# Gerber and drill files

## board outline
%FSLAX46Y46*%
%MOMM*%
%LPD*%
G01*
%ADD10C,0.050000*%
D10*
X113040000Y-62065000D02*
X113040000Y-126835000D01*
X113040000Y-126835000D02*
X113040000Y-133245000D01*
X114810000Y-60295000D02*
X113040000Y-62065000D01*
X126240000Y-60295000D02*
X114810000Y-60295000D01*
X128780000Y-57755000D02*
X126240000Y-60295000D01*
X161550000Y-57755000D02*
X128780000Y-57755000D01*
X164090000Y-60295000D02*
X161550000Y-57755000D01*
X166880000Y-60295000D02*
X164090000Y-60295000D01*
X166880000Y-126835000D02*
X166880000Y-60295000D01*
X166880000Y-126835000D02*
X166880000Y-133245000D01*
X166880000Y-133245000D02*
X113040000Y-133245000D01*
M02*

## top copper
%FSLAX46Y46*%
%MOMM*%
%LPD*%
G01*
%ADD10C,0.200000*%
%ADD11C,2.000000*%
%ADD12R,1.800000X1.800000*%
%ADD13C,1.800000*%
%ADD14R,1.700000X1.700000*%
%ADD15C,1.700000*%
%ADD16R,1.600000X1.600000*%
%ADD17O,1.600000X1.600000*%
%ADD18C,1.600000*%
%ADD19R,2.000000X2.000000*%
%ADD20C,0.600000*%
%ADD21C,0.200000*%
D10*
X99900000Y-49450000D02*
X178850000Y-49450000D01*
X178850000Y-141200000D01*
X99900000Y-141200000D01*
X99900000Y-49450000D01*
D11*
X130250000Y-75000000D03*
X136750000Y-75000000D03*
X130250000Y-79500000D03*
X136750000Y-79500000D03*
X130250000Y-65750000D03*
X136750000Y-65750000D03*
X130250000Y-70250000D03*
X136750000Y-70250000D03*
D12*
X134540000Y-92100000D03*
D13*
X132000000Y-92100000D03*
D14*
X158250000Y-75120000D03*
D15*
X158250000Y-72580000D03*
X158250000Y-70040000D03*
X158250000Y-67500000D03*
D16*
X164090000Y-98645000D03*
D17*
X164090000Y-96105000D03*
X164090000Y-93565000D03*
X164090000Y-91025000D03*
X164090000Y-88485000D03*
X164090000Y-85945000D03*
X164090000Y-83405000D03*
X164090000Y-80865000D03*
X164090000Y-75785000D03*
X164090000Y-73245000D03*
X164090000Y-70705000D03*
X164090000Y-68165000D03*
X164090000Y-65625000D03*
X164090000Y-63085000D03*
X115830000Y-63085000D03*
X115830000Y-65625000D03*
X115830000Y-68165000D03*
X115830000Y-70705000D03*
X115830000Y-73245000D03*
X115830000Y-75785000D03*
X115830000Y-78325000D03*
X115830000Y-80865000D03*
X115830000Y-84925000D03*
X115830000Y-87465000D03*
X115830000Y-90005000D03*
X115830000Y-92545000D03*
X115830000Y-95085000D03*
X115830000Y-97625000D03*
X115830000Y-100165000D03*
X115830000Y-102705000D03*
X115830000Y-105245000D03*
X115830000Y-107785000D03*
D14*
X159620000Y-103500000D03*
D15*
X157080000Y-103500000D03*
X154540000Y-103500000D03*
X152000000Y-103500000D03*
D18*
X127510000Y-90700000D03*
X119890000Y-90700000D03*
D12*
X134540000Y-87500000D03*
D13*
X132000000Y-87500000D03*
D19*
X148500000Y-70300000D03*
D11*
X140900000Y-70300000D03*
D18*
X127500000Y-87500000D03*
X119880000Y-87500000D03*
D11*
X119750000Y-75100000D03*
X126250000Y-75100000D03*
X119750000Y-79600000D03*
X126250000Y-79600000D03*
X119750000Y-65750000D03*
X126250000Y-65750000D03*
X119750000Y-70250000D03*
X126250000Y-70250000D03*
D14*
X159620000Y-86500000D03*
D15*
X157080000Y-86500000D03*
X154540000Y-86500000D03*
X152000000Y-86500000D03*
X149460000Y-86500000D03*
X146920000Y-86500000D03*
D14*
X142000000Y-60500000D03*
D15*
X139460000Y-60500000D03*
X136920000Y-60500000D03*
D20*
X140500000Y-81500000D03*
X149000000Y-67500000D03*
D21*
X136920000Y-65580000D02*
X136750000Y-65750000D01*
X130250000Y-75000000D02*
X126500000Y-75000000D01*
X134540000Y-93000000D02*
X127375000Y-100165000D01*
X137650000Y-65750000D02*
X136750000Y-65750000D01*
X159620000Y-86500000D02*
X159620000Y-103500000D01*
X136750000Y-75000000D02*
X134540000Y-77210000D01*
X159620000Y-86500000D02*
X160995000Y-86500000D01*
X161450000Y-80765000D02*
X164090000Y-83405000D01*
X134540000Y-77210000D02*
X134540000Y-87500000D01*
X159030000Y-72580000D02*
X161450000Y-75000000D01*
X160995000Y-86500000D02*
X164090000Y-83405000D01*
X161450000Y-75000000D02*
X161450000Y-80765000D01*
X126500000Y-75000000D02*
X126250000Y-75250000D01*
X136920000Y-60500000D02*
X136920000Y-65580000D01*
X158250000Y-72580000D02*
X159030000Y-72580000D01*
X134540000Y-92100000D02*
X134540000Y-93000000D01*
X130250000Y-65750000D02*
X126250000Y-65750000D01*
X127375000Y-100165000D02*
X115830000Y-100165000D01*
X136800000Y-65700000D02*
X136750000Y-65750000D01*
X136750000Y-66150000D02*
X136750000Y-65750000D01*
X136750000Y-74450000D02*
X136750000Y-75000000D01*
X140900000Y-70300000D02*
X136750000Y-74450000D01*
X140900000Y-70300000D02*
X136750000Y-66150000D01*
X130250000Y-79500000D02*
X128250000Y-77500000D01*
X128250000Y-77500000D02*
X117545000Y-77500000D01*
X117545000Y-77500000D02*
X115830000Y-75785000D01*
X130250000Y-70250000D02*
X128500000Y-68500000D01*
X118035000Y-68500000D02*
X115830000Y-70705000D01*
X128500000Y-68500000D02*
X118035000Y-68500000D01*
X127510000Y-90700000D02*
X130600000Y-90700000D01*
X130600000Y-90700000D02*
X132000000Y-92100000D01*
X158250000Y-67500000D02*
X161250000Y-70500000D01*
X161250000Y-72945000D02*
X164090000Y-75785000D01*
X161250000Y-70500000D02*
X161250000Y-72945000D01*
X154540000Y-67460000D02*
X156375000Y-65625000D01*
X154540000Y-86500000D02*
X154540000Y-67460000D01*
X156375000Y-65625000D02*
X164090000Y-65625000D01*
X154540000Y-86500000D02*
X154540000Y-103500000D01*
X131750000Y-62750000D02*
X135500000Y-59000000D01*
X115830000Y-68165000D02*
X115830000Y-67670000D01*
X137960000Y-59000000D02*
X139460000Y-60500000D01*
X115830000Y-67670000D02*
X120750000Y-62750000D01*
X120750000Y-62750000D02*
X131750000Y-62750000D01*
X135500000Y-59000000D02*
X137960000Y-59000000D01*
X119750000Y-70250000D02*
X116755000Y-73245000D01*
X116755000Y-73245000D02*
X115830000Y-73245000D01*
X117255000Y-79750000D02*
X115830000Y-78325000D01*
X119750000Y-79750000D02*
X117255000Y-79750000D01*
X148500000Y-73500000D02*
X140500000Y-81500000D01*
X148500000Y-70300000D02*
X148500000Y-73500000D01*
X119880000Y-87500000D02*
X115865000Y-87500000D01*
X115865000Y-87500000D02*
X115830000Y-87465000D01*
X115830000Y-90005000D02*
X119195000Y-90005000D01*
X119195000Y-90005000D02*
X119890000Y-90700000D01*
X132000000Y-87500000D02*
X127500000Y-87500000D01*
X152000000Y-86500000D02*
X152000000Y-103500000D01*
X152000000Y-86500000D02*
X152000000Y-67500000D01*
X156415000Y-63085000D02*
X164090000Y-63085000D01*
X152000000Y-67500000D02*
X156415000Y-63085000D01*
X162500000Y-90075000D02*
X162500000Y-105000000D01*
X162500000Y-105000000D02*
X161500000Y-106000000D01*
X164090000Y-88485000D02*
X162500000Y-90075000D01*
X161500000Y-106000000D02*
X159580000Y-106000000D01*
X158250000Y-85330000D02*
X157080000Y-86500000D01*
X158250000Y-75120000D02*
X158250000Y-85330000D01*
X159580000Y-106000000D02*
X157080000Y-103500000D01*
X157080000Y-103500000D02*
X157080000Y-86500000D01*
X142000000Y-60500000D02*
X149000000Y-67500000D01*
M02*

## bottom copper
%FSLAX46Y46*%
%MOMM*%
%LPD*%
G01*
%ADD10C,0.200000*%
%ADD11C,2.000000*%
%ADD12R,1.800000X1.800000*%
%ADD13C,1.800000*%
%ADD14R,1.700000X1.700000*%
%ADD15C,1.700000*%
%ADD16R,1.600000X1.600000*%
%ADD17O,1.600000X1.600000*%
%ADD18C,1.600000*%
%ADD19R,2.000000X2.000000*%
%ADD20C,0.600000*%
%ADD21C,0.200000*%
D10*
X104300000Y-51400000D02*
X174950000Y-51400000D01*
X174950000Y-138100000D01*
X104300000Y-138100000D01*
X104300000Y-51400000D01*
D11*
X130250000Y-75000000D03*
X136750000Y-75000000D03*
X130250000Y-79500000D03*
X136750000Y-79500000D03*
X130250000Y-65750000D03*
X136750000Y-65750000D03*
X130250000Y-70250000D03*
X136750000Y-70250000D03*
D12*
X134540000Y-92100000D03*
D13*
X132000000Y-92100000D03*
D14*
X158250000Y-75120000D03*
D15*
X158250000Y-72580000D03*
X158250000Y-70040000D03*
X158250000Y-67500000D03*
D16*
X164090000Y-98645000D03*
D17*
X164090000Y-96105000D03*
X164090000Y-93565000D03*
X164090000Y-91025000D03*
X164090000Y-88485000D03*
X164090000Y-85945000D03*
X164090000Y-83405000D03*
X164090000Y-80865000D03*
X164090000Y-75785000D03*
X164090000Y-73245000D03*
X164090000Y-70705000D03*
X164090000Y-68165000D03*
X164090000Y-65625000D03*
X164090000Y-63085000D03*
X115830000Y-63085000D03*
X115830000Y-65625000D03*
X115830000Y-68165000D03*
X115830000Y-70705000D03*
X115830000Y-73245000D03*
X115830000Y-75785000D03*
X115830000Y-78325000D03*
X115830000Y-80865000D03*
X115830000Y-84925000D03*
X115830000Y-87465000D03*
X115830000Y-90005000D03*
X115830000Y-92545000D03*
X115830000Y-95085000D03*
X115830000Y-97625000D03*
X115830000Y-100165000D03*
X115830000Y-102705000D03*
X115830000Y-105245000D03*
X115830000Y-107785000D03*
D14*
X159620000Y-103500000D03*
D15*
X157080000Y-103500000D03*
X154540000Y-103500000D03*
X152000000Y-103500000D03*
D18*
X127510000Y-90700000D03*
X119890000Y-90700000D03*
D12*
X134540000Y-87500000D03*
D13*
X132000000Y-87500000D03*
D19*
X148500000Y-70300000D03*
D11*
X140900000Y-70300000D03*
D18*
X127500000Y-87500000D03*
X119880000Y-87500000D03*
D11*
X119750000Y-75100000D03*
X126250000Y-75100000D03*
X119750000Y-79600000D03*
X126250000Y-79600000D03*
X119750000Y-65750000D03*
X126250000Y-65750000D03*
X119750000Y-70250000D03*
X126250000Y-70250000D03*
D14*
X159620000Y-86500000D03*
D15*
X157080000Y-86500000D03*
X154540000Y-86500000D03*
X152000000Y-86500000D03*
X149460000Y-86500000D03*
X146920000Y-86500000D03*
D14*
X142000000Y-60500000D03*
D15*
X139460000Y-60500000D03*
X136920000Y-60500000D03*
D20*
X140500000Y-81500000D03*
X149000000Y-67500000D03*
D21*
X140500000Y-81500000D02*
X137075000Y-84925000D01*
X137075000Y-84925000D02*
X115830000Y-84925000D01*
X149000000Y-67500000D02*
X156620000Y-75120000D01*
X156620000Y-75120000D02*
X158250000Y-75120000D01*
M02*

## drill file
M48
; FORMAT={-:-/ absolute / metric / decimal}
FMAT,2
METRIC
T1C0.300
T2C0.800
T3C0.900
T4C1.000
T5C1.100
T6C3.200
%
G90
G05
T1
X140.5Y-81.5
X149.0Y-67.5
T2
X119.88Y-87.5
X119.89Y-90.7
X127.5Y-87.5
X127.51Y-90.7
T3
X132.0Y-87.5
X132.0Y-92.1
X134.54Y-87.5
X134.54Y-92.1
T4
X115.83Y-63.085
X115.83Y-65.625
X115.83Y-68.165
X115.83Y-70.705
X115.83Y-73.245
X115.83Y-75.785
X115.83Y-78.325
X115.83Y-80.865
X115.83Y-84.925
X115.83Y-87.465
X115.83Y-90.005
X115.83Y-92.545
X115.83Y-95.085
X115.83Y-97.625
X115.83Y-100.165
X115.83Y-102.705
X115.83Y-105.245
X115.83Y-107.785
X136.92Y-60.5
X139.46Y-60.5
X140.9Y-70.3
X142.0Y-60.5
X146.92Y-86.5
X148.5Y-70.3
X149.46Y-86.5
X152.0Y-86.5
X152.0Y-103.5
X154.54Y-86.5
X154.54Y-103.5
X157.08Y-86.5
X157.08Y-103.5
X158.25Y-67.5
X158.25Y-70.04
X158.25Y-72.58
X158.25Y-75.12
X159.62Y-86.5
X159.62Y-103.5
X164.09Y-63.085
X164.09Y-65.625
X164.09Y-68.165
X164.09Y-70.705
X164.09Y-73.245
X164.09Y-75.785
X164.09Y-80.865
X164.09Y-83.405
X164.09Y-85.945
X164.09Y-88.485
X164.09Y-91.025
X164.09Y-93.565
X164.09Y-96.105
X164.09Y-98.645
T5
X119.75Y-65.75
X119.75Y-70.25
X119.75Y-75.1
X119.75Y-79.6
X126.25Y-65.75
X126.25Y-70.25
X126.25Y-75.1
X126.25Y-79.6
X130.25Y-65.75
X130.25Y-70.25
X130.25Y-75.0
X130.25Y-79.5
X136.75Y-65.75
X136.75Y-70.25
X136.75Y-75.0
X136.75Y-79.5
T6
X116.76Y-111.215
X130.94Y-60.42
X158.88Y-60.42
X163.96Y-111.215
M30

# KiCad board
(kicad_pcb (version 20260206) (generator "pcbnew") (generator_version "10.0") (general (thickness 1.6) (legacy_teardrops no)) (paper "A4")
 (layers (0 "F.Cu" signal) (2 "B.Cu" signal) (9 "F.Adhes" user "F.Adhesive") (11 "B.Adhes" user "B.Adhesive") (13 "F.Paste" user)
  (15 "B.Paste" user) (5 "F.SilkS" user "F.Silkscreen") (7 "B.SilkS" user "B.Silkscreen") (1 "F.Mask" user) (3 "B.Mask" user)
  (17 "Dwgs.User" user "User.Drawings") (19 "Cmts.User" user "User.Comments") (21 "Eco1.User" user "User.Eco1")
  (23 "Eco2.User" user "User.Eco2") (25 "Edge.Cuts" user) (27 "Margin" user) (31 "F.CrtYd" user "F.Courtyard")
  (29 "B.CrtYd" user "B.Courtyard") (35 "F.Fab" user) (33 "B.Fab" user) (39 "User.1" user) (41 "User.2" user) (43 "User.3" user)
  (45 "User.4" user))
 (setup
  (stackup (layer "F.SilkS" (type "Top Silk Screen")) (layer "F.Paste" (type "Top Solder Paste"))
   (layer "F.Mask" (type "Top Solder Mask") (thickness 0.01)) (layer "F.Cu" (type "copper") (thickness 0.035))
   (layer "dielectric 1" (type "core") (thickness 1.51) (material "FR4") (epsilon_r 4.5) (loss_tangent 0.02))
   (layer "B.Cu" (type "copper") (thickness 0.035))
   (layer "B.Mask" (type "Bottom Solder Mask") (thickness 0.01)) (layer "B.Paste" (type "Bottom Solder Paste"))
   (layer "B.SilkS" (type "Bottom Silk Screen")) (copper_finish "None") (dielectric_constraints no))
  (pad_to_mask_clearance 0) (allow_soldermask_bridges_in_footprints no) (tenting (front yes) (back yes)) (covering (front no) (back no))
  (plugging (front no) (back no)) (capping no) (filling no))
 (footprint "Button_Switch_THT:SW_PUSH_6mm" (layer "F.Cu") (at 130.25 75)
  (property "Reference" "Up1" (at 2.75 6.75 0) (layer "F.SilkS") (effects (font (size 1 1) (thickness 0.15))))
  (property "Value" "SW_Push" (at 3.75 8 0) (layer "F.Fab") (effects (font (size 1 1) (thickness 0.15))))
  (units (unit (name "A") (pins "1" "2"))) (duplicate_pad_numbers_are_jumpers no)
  (pad "1" thru_hole circle (at 0 0 90) (size 2 2) (drill 1.1) (layers "*.Cu" "*.Mask") (remove_unused_layers no) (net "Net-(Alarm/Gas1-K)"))
  (pad "1" thru_hole circle (at 6.5 0 90) (size 2 2) (drill 1.1) (layers "*.Cu" "*.Mask") (remove_unused_layers no)
   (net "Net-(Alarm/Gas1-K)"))
  (pad "2" thru_hole circle (at 0 4.5 90) (size 2 2) (drill 1.1) (layers "*.Cu" "*.Mask") (remove_unused_layers no) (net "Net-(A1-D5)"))
  (pad "2" thru_hole circle (at 6.5 4.5 90) (size 2 2) (drill 1.1) (layers "*.Cu" "*.Mask") (remove_unused_layers no) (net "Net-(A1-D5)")))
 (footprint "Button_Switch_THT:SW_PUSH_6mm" (layer "F.Cu") (at 130.25 65.75)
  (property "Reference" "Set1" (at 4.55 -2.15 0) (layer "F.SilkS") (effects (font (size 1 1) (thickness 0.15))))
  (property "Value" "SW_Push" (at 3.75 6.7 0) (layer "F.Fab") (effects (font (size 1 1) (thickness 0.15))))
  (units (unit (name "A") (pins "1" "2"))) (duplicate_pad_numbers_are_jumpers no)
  (pad "1" thru_hole circle (at 0 0 90) (size 2 2) (drill 1.1) (layers "*.Cu" "*.Mask") (remove_unused_layers no) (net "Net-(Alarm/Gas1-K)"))
  (pad "1" thru_hole circle (at 6.5 0 90) (size 2 2) (drill 1.1) (layers "*.Cu" "*.Mask") (remove_unused_layers no)
   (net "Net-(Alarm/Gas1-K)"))
  (pad "2" thru_hole circle (at 0 4.5 90) (size 2 2) (drill 1.1) (layers "*.Cu" "*.Mask") (remove_unused_layers no) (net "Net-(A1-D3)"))
  (pad "2" thru_hole circle (at 6.5 4.5 90) (size 2 2) (drill 1.1) (layers "*.Cu" "*.Mask") (remove_unused_layers no) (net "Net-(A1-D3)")))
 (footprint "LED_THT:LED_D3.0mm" (layer "F.Cu") (at 134.54 92.1 180)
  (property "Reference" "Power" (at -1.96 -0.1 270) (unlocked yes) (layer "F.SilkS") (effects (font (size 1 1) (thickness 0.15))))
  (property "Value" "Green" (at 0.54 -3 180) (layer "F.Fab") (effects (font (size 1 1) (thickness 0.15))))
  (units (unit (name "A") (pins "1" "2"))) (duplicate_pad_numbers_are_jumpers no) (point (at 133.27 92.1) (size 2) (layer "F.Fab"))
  (pad "1" thru_hole rect (at 0 0 180) (size 1.8 1.8) (drill 0.9) (layers "*.Cu" "*.Mask") (remove_unused_layers no)
   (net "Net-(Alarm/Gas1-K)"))
  (pad "2" thru_hole circle (at 2.54 0 180) (size 1.8 1.8) (drill 0.9) (layers "*.Cu" "*.Mask") (remove_unused_layers no)
   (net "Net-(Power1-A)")))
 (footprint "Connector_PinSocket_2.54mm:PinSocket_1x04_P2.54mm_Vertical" (layer "F.Cu") (at 158.25 75.12 180)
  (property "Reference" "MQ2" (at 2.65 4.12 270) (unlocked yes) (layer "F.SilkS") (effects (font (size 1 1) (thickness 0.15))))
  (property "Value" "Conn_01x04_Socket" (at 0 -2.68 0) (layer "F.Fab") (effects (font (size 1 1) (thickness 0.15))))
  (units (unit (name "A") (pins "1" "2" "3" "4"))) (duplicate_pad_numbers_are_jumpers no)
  (pad "1" thru_hole rect (at 0 0 180) (size 1.7 1.7) (drill 1) (layers "*.Cu" "*.Mask") (remove_unused_layers no) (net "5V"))
  (pad "2" thru_hole circle (at 0 2.54 180) (size 1.7 1.7) (drill 1) (layers "*.Cu" "*.Mask") (remove_unused_layers no)
   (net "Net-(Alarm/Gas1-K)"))
  (pad "3" thru_hole circle (at 0 5.08 180) (size 1.7 1.7) (drill 1) (layers "*.Cu" "*.Mask") (remove_unused_layers no)
   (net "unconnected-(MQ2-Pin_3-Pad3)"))
  (pad "4" thru_hole circle (at 0 7.62 180) (size 1.7 1.7) (drill 1) (layers "*.Cu" "*.Mask") (remove_unused_layers no) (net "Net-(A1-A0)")))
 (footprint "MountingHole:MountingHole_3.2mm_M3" (layer "F.Cu") (at 163.96 111.215)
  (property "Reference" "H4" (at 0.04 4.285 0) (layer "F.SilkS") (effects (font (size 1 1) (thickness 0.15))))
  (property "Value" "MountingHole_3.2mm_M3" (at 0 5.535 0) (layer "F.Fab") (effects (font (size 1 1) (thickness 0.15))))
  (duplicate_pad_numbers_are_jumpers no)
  (pad "" np_thru_hole circle (at 0 0) (size 3.2 3.2) (drill 3.2) (layers "*.Cu" "*.Mask")))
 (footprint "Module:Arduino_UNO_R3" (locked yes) (layer "F.Cu") (at 116.09 98.645 90)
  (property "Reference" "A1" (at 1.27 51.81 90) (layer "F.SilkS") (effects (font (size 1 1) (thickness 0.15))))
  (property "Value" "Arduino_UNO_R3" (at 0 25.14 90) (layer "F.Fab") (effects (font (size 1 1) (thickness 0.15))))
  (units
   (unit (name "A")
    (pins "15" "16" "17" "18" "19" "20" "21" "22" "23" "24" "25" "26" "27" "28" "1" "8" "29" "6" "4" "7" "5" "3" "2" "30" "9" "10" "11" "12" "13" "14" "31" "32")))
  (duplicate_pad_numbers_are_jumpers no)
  (fp_line (start 36.58 -3.05) (end -28.19 -3.05) (stroke (width 0.05) (type solid)) (layer "Edge.Cuts"))
  (fp_line (start -28.19 -3.05) (end -34.6 -3.05) (stroke (width 0.05) (type default)) (layer "Edge.Cuts"))
  (fp_line (start 38.35 -1.28) (end 36.58 -3.05) (stroke (width 0.05) (type solid)) (layer "Edge.Cuts"))
  (fp_line (start 38.35 10.15) (end 38.35 -1.28) (stroke (width 0.05) (type solid)) (layer "Edge.Cuts"))
  (fp_line (start 40.89 12.69) (end 38.35 10.15) (stroke (width 0.05) (type solid)) (layer "Edge.Cuts"))
  (fp_line (start 40.89 45.46) (end 40.89 12.69) (stroke (width 0.05) (type solid)) (layer "Edge.Cuts"))
  (fp_line (start 38.35 48) (end 40.89 45.46) (stroke (width 0.05) (type solid)) (layer "Edge.Cuts"))
  (fp_line (start 38.35 50.79) (end 38.35 48) (stroke (width 0.05) (type solid)) (layer "Edge.Cuts"))
  (fp_line (start -28.19 50.79) (end 38.35 50.79) (stroke (width 0.05) (type solid)) (layer "Edge.Cuts"))
  (fp_line (start -28.19 50.79) (end -34.6 50.79) (stroke (width 0.05) (type default)) (layer "Edge.Cuts"))
  (fp_line (start -34.6 50.79) (end -34.6 -3.05) (stroke (width 0.05) (type default)) (layer "Edge.Cuts"))
  (pad "1" thru_hole rect (at 0 48) (size 1.6 1.6) (drill 1) (layers "*.Cu" "*.Mask") (remove_unused_layers no)
   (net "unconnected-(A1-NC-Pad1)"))
  (pad "2" thru_hole oval (at 2.54 48) (size 1.6 1.6) (drill 1) (layers "*.Cu" "*.Mask") (remove_unused_layers no)
   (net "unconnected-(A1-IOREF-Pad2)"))
  (pad "3" thru_hole oval (at 5.08 48) (size 1.6 1.6) (drill 1) (layers "*.Cu" "*.Mask") (remove_unused_layers no)
   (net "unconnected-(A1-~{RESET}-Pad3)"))
  (pad "4" thru_hole oval (at 7.62 48) (size 1.6 1.6) (drill 1) (layers "*.Cu" "*.Mask") (remove_unused_layers no)
   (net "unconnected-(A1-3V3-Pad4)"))
  (pad "5" thru_hole oval (at 10.16 48) (size 1.6 1.6) (drill 1) (layers "*.Cu" "*.Mask") (remove_unused_layers no) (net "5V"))
  (pad "6" thru_hole oval (at 12.7 48) (size 1.6 1.6) (drill 1) (layers "*.Cu" "*.Mask") (remove_unused_layers no) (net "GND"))
  (pad "7" thru_hole oval (at 15.24 48) (size 1.6 1.6) (drill 1) (layers "*.Cu" "*.Mask") (remove_unused_layers no)
   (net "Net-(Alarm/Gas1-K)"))
  (pad "8" thru_hole oval (at 17.78 48) (size 1.6 1.6) (drill 1) (layers "*.Cu" "*.Mask") (remove_unused_layers no)
   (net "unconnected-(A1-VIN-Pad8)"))
  (pad "9" thru_hole oval (at 22.86 48) (size 1.6 1.6) (drill 1) (layers "*.Cu" "*.Mask") (remove_unused_layers no) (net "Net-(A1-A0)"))
  (pad "10" thru_hole oval (at 25.4 48) (size 1.6 1.6) (drill 1) (layers "*.Cu" "*.Mask") (remove_unused_layers no)
   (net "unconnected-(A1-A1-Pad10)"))
  (pad "11" thru_hole oval (at 27.94 48) (size 1.6 1.6) (drill 1) (layers "*.Cu" "*.Mask") (remove_unused_layers no)
   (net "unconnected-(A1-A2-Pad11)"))
  (pad "12" thru_hole oval (at 30.48 48) (size 1.6 1.6) (drill 1) (layers "*.Cu" "*.Mask") (remove_unused_layers no)
   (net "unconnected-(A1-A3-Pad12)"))
  (pad "13" thru_hole oval (at 33.02 48) (size 1.6 1.6) (drill 1) (layers "*.Cu" "*.Mask") (remove_unused_layers no)
   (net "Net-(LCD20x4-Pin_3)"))
  (pad "14" thru_hole oval (at 35.56 48) (size 1.6 1.6) (drill 1) (layers "*.Cu" "*.Mask") (remove_unused_layers no)
   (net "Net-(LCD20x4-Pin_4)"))
  (pad "15" thru_hole oval (at 35.56 -0.26) (size 1.6 1.6) (drill 1) (layers "*.Cu" "*.Mask") (remove_unused_layers no)
   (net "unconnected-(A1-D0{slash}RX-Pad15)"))
  (pad "16" thru_hole oval (at 33.02 -0.26) (size 1.6 1.6) (drill 1) (layers "*.Cu" "*.Mask") (remove_unused_layers no)
   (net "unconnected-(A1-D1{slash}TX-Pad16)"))
  (pad "17" thru_hole oval (at 30.48 -0.26) (size 1.6 1.6) (drill 1) (layers "*.Cu" "*.Mask") (remove_unused_layers no) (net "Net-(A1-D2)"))
  (pad "18" thru_hole oval (at 27.94 -0.26) (size 1.6 1.6) (drill 1) (layers "*.Cu" "*.Mask") (remove_unused_layers no) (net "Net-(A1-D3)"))
  (pad "19" thru_hole oval (at 25.4 -0.26) (size 1.6 1.6) (drill 1) (layers "*.Cu" "*.Mask") (remove_unused_layers no) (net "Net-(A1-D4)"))
  (pad "20" thru_hole oval (at 22.86 -0.26) (size 1.6 1.6) (drill 1) (layers "*.Cu" "*.Mask") (remove_unused_layers no) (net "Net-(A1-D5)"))
  (pad "21" thru_hole oval (at 20.32 -0.26) (size 1.6 1.6) (drill 1) (layers "*.Cu" "*.Mask") (remove_unused_layers no) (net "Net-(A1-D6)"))
  (pad "22" thru_hole oval (at 17.78 -0.26) (size 1.6 1.6) (drill 1) (layers "*.Cu" "*.Mask") (remove_unused_layers no)
   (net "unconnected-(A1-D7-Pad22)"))
  (pad "23" thru_hole oval (at 13.72 -0.26) (size 1.6 1.6) (drill 1) (layers "*.Cu" "*.Mask") (remove_unused_layers no) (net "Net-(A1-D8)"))
  (pad "24" thru_hole oval (at 11.18 -0.26) (size 1.6 1.6) (drill 1) (layers "*.Cu" "*.Mask") (remove_unused_layers no) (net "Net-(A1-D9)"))
  (pad "25" thru_hole oval (at 8.64 -0.26) (size 1.6 1.6) (drill 1) (layers "*.Cu" "*.Mask") (remove_unused_layers no) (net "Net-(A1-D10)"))
  (pad "26" thru_hole oval (at 6.1 -0.26) (size 1.6 1.6) (drill 1) (layers "*.Cu" "*.Mask") (remove_unused_layers no)
   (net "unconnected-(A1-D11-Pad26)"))
  (pad "27" thru_hole oval (at 3.56 -0.26) (size 1.6 1.6) (drill 1) (layers "*.Cu" "*.Mask") (remove_unused_layers no)
   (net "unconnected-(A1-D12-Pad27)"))
  (pad "28" thru_hole oval (at 1.02 -0.26) (size 1.6 1.6) (drill 1) (layers "*.Cu" "*.Mask") (remove_unused_layers no)
   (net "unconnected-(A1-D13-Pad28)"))
  (pad "29" thru_hole oval (at -1.52 -0.26) (size 1.6 1.6) (drill 1) (layers "*.Cu" "*.Mask") (remove_unused_layers no)
   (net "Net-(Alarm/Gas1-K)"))
  (pad "30" thru_hole oval (at -4.06 -0.26) (size 1.6 1.6) (drill 1) (layers "*.Cu" "*.Mask") (remove_unused_layers no)
   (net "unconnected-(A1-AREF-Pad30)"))
  (pad "31" thru_hole oval (at -6.6 -0.26) (size 1.6 1.6) (drill 1) (layers "*.Cu" "*.Mask") (remove_unused_layers no)
   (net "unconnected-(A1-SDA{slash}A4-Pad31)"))
  (pad "32" thru_hole oval (at -9.14 -0.26) (size 1.6 1.6) (drill 1) (layers "*.Cu" "*.Mask") (remove_unused_layers no)
   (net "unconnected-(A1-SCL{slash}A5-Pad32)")))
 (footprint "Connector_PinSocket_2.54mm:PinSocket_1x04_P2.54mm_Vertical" (layer "F.Cu") (at 159.62 103.5 -90)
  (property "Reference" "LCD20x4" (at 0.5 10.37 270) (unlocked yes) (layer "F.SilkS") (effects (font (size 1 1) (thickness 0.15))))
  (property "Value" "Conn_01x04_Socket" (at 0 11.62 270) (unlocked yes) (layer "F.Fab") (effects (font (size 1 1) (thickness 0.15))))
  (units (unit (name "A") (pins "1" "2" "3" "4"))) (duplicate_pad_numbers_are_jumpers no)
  (pad "1" thru_hole rect (at 0 0 270) (size 1.7 1.7) (drill 1) (layers "*.Cu" "*.Mask") (remove_unused_layers no)
   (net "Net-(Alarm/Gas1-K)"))
  (pad "2" thru_hole circle (at 0 2.54 270) (size 1.7 1.7) (drill 1) (layers "*.Cu" "*.Mask") (remove_unused_layers no) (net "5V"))
  (pad "3" thru_hole circle (at 0 5.08 270) (size 1.7 1.7) (drill 1) (layers "*.Cu" "*.Mask") (remove_unused_layers no)
   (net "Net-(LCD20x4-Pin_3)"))
  (pad "4" thru_hole circle (at 0 7.62 270) (size 1.7 1.7) (drill 1) (layers "*.Cu" "*.Mask") (remove_unused_layers no)
   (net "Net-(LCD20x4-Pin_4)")))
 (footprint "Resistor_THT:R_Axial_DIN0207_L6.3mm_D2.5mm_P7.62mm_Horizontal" (layer "F.Cu") (at 127.51 90.7 180)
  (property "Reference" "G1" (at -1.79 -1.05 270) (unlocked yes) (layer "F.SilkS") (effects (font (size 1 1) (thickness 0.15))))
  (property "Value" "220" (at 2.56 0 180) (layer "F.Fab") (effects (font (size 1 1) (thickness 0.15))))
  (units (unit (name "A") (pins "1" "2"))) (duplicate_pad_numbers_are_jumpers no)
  (pad "1" thru_hole circle (at 0 0 180) (size 1.6 1.6) (drill 0.8) (layers "*.Cu" "*.Mask") (remove_unused_layers no)
   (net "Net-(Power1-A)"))
  (pad "2" thru_hole circle (at 7.62 0 180) (size 1.6 1.6) (drill 0.8) (layers "*.Cu" "*.Mask") (remove_unused_layers no)
   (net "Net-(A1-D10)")))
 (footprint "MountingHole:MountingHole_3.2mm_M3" (layer "F.Cu") (at 116.76 111.215)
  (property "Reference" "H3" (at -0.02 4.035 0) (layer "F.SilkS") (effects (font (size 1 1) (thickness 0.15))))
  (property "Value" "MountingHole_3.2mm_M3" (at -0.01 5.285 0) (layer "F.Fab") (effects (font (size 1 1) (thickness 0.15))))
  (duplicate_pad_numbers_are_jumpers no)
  (pad "" np_thru_hole circle (at 0 0) (size 3.2 3.2) (drill 3.2) (layers "*.Cu" "*.Mask")))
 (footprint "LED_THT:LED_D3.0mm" (layer "F.Cu") (at 134.54 87.5 180)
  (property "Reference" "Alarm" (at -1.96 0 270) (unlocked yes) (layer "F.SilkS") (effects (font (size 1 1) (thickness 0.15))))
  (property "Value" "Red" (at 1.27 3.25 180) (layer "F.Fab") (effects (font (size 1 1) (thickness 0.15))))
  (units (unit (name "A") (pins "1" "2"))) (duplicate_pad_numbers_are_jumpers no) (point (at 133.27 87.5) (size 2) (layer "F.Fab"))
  (pad "1" thru_hole rect (at 0 0 180) (size 1.8 1.8) (drill 0.9) (layers "*.Cu" "*.Mask") (remove_unused_layers no)
   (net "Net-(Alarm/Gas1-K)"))
  (pad "2" thru_hole circle (at 2.54 0 180) (size 1.8 1.8) (drill 0.9) (layers "*.Cu" "*.Mask") (remove_unused_layers no)
   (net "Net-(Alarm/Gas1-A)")))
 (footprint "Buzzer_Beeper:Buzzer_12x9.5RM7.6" (layer "F.Cu") (at 148.5 70.3 180)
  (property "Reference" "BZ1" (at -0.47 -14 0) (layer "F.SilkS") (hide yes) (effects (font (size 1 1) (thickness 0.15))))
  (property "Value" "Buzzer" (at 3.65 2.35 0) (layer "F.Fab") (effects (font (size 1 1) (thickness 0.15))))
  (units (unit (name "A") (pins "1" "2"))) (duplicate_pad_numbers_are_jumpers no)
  (pad "1" thru_hole rect (at 0 0 180) (size 2 2) (drill 1) (layers "*.Cu" "*.Mask") (remove_unused_layers no) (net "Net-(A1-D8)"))
  (pad "2" thru_hole circle (at 7.6 0 180) (size 2 2) (drill 1) (layers "*.Cu" "*.Mask") (remove_unused_layers no)
   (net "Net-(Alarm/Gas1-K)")))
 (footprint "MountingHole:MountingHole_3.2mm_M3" (layer "F.Cu") (at 158.88 60.42)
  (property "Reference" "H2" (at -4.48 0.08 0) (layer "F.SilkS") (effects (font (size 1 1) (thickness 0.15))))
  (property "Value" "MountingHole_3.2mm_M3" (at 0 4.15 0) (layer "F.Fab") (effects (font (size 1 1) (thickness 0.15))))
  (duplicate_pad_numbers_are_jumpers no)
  (pad "" np_thru_hole circle (at 0 0) (size 3.2 3.2) (drill 3.2) (layers "*.Cu" "*.Mask")))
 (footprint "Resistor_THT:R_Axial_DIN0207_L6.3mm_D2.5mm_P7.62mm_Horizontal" (layer "F.Cu") (at 127.5 87.5 180)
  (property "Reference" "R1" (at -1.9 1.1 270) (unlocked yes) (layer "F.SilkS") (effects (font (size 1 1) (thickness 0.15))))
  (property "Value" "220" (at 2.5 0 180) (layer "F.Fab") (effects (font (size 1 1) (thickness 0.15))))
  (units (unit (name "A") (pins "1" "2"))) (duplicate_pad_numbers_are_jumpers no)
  (pad "1" thru_hole circle (at 0 0 180) (size 1.6 1.6) (drill 0.8) (layers "*.Cu" "*.Mask") (remove_unused_layers no)
   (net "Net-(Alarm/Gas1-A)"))
  (pad "2" thru_hole circle (at 7.62 0 180) (size 1.6 1.6) (drill 0.8) (layers "*.Cu" "*.Mask") (remove_unused_layers no)
   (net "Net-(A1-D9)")))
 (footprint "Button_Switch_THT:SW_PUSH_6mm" (layer "F.Cu") (at 119.75 75.1)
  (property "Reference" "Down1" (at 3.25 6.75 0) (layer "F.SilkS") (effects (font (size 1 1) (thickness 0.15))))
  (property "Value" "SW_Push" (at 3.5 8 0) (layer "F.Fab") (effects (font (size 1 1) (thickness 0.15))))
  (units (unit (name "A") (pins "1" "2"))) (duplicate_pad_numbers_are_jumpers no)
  (pad "1" thru_hole circle (at 0 0 90) (size 2 2) (drill 1.1) (layers "*.Cu" "*.Mask") (remove_unused_layers no) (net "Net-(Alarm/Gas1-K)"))
  (pad "1" thru_hole circle (at 6.5 0 90) (size 2 2) (drill 1.1) (layers "*.Cu" "*.Mask") (remove_unused_layers no)
   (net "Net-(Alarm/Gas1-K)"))
  (pad "2" thru_hole circle (at 0 4.5 90) (size 2 2) (drill 1.1) (layers "*.Cu" "*.Mask") (remove_unused_layers no) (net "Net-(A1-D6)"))
  (pad "2" thru_hole circle (at 6.5 4.5 90) (size 2 2) (drill 1.1) (layers "*.Cu" "*.Mask") (remove_unused_layers no) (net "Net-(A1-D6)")))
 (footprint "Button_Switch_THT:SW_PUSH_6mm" (layer "F.Cu") (at 119.75 65.75)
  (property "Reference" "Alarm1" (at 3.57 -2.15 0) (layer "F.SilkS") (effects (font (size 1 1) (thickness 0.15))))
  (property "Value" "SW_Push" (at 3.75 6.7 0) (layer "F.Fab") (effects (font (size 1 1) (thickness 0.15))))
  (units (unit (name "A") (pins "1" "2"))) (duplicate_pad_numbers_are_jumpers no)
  (pad "1" thru_hole circle (at 0 0 90) (size 2 2) (drill 1.1) (layers "*.Cu" "*.Mask") (remove_unused_layers no) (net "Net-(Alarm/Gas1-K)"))
  (pad "1" thru_hole circle (at 6.5 0 90) (size 2 2) (drill 1.1) (layers "*.Cu" "*.Mask") (remove_unused_layers no)
   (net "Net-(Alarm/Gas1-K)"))
  (pad "2" thru_hole circle (at 0 4.5 90) (size 2 2) (drill 1.1) (layers "*.Cu" "*.Mask") (remove_unused_layers no) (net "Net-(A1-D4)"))
  (pad "2" thru_hole circle (at 6.5 4.5 90) (size 2 2) (drill 1.1) (layers "*.Cu" "*.Mask") (remove_unused_layers no) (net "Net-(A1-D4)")))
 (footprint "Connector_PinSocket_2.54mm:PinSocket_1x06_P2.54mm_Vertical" (layer "F.Cu") (at 159.62 86.5 -90)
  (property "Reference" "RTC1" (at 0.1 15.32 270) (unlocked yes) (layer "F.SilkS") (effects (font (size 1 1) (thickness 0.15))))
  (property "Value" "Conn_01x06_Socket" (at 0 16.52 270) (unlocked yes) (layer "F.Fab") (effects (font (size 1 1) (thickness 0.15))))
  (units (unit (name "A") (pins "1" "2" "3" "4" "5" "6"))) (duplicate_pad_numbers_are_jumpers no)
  (pad "1" thru_hole rect (at 0 0 270) (size 1.7 1.7) (drill 1) (layers "*.Cu" "*.Mask") (remove_unused_layers no)
   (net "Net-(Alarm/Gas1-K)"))
  (pad "2" thru_hole circle (at 0 2.54 270) (size 1.7 1.7) (drill 1) (layers "*.Cu" "*.Mask") (remove_unused_layers no) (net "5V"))
  (pad "3" thru_hole circle (at 0 5.08 270) (size 1.7 1.7) (drill 1) (layers "*.Cu" "*.Mask") (remove_unused_layers no)
   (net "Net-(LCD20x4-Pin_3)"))
  (pad "4" thru_hole circle (at 0 7.62 270) (size 1.7 1.7) (drill 1) (layers "*.Cu" "*.Mask") (remove_unused_layers no)
   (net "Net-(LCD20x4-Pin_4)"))
  (pad "5" thru_hole circle (at 0 10.16 270) (size 1.7 1.7) (drill 1) (layers "*.Cu" "*.Mask") (remove_unused_layers no)
   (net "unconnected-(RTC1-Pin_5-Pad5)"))
  (pad "6" thru_hole circle (at 0 12.7 270) (size 1.7 1.7) (drill 1) (layers "*.Cu" "*.Mask") (remove_unused_layers no)
   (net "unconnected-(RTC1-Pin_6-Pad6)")))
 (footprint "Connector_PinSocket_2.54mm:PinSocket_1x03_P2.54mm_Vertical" (layer "F.Cu") (at 142 60.5 -90)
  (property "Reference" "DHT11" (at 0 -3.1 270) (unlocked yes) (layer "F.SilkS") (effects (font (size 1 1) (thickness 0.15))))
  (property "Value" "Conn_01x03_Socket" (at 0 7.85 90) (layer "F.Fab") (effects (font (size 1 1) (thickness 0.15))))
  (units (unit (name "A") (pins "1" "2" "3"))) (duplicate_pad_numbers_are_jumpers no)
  (pad "1" thru_hole rect (at 0 0 270) (size 1.7 1.7) (drill 1) (layers "*.Cu" "*.Mask") (remove_unused_layers no) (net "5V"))
  (pad "2" thru_hole circle (at 0 2.54 270) (size 1.7 1.7) (drill 1) (layers "*.Cu" "*.Mask") (remove_unused_layers no) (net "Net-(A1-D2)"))
  (pad "3" thru_hole circle (at 0 5.08 270) (size 1.7 1.7) (drill 1) (layers "*.Cu" "*.Mask") (remove_unused_layers no)
   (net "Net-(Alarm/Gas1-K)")))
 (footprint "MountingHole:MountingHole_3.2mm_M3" (layer "F.Cu") (at 130.94 60.42)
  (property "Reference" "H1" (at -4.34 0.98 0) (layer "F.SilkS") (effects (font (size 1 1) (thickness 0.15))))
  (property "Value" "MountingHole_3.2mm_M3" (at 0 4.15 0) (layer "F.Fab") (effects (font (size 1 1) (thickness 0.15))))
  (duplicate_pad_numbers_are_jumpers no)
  (pad "" np_thru_hole circle (at 0 0) (size 3.2 3.2) (drill 3.2) (layers "*.Cu" "*.Mask")))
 (gr_rect (start 99.9 49.45) (end 178.85 141.2) (stroke (width 0.2) (type default)) (fill no) (layers "F.Cu" "F.Mask"))
 (gr_rect (start 104.3 51.4) (end 174.95 138.1) (stroke (width 0.2) (type default)) (fill no) (layer "B.Cu"))
 (segment (start 136.92 65.58) (end 136.75 65.75) (width 0.2) (layer "F.Cu") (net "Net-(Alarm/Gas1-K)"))
 (segment (start 130.25 75) (end 126.5 75) (width 0.2) (layer "F.Cu") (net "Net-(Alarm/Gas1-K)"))
 (segment (start 134.54 93) (end 127.375 100.165) (width 0.2) (layer "F.Cu") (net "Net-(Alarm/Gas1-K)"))
 (segment (start 137.65 65.75) (end 136.75 65.75) (width 0.2) (layer "F.Cu") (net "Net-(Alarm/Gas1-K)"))
 (segment (start 159.62 86.5) (end 159.62 103.5) (width 0.2) (layer "F.Cu") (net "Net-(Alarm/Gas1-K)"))
 (segment (start 136.75 75) (end 134.54 77.21) (width 0.2) (layer "F.Cu") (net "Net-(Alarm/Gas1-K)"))
 (segment (start 159.62 86.5) (end 160.995 86.5) (width 0.2) (layer "F.Cu") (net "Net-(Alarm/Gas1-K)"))
 (segment (start 161.45 80.765) (end 164.09 83.405) (width 0.2) (layer "F.Cu") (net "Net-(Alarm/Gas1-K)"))
 (segment (start 134.54 77.21) (end 134.54 87.5) (width 0.2) (layer "F.Cu") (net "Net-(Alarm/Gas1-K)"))
 (segment (start 159.03 72.58) (end 161.45 75) (width 0.2) (layer "F.Cu") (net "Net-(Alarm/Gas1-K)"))
 (segment (start 160.995 86.5) (end 164.09 83.405) (width 0.2) (layer "F.Cu") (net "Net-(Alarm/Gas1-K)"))
 (segment (start 161.45 75) (end 161.45 80.765) (width 0.2) (layer "F.Cu") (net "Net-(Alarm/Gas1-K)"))
 (segment (start 126.5 75) (end 126.25 75.25) (width 0.2) (layer "F.Cu") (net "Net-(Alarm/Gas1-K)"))
 (segment (start 136.92 60.5) (end 136.92 65.58) (width 0.2) (layer "F.Cu") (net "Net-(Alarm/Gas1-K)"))
 (segment (start 158.25 72.58) (end 159.03 72.58) (width 0.2) (layer "F.Cu") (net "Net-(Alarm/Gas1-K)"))
 (segment (start 134.54 92.1) (end 134.54 93) (width 0.2) (layer "F.Cu") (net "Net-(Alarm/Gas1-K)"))
 (segment (start 130.25 65.75) (end 126.25 65.75) (width 0.2) (layer "F.Cu") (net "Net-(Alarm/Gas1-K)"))
 (segment (start 127.375 100.165) (end 115.83 100.165) (width 0.2) (layer "F.Cu") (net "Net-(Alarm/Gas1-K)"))
 (segment (start 136.8 65.7) (end 136.75 65.75) (width 0.2) (layer "F.Cu") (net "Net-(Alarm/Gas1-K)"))
 (segment (start 136.75 66.15) (end 136.75 65.75) (width 0.2) (layer "F.Cu") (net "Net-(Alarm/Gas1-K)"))
 (segment (start 136.75 74.45) (end 136.75 75) (width 0.2) (layer "F.Cu") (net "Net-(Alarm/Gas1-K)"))
 (segment (start 140.9 70.3) (end 136.75 74.45) (width 0.2) (layer "F.Cu") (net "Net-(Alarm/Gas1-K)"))
 (segment (start 140.9 70.3) (end 136.75 66.15) (width 0.2) (layer "F.Cu") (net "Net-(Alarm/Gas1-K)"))
 (segment (start 130.25 79.5) (end 128.25 77.5) (width 0.2) (layer "F.Cu") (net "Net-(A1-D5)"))
 (segment (start 128.25 77.5) (end 117.545 77.5) (width 0.2) (layer "F.Cu") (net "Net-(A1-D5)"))
 (segment (start 117.545 77.5) (end 115.83 75.785) (width 0.2) (layer "F.Cu") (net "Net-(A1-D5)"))
 (segment (start 130.25 70.25) (end 128.5 68.5) (width 0.2) (layer "F.Cu") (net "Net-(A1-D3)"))
 (segment (start 118.035 68.5) (end 115.83 70.705) (width 0.2) (layer "F.Cu") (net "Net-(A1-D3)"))
 (segment (start 128.5 68.5) (end 118.035 68.5) (width 0.2) (layer "F.Cu") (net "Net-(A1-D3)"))
 (segment (start 127.51 90.7) (end 130.6 90.7) (width 0.2) (layer "F.Cu") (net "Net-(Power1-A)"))
 (segment (start 130.6 90.7) (end 132 92.1) (width 0.2) (layer "F.Cu") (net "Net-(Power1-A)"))
 (segment (start 158.25 67.5) (end 161.25 70.5) (width 0.2) (layer "F.Cu") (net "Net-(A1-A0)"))
 (segment (start 161.25 72.945) (end 164.09 75.785) (width 0.2) (layer "F.Cu") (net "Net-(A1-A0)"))
 (segment (start 161.25 70.5) (end 161.25 72.945) (width 0.2) (layer "F.Cu") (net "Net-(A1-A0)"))
 (segment (start 154.54 67.46) (end 156.375 65.625) (width 0.2) (layer "F.Cu") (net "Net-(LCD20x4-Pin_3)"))
 (segment (start 154.54 86.5) (end 154.54 67.46) (width 0.2) (layer "F.Cu") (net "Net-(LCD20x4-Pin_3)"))
 (segment (start 156.375 65.625) (end 164.09 65.625) (width 0.2) (layer "F.Cu") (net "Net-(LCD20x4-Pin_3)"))
 (segment (start 154.54 86.5) (end 154.54 103.5) (width 0.2) (layer "F.Cu") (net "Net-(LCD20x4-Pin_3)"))
 (segment (start 131.75 62.75) (end 135.5 59) (width 0.2) (layer "F.Cu") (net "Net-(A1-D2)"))
 (segment (start 115.83 68.165) (end 115.83 67.67) (width 0.2) (layer "F.Cu") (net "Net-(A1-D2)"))
 (segment (start 137.96 59) (end 139.46 60.5) (width 0.2) (layer "F.Cu") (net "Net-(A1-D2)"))
 (segment (start 115.83 67.67) (end 120.75 62.75) (width 0.2) (layer "F.Cu") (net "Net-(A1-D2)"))
 (segment (start 120.75 62.75) (end 131.75 62.75) (width 0.2) (layer "F.Cu") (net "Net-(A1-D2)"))
 (segment (start 135.5 59) (end 137.96 59) (width 0.2) (layer "F.Cu") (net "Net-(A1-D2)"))
 (segment (start 119.75 70.25) (end 116.755 73.245) (width 0.2) (layer "F.Cu") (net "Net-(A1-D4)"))
 (segment (start 116.755 73.245) (end 115.83 73.245) (width 0.2) (layer "F.Cu") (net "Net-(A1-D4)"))
 (segment (start 117.255 79.75) (end 115.83 78.325) (width 0.2) (layer "F.Cu") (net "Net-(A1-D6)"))
 (segment (start 119.75 79.75) (end 117.255 79.75) (width 0.2) (layer "F.Cu") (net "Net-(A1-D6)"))
 (segment (start 148.5 73.5) (end 140.5 81.5) (width 0.2) (layer "F.Cu") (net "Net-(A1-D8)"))
 (segment (start 148.5 70.3) (end 148.5 73.5) (width 0.2) (layer "F.Cu") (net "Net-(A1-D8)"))
 (via (at 140.5 81.5) (size 0.6) (drill 0.3) (layers "F.Cu" "B.Cu") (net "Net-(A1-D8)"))
 (segment (start 140.5 81.5) (end 137.075 84.925) (width 0.2) (layer "B.Cu") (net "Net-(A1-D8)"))
 (segment (start 137.075 84.925) (end 115.83 84.925) (width 0.2) (layer "B.Cu") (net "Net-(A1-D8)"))
 (segment (start 119.88 87.5) (end 115.865 87.5) (width 0.2) (layer "F.Cu") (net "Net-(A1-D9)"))
 (segment (start 115.865 87.5) (end 115.83 87.465) (width 0.2) (layer "F.Cu") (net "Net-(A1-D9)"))
 (segment (start 115.83 90.005) (end 119.195 90.005) (width 0.2) (layer "F.Cu") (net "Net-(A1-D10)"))
 (segment (start 119.195 90.005) (end 119.89 90.7) (width 0.2) (layer "F.Cu") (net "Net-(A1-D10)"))
 (segment (start 132 87.5) (end 127.5 87.5) (width 0.2) (layer "F.Cu") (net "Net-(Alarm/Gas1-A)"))
 (segment (start 152 86.5) (end 152 103.5) (width 0.2) (layer "F.Cu") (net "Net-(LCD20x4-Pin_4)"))
 (segment (start 152 86.5) (end 152 67.5) (width 0.2) (layer "F.Cu") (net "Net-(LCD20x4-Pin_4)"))
 (segment (start 156.415 63.085) (end 164.09 63.085) (width 0.2) (layer "F.Cu") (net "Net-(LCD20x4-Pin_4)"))
 (segment (start 152 67.5) (end 156.415 63.085) (width 0.2) (layer "F.Cu") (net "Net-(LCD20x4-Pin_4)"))
 (segment (start 162.5 90.075) (end 162.5 105) (width 0.2) (layer "F.Cu") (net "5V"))
 (segment (start 162.5 105) (end 161.5 106) (width 0.2) (layer "F.Cu") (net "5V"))
 (segment (start 164.09 88.485) (end 162.5 90.075) (width 0.2) (layer "F.Cu") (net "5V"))
 (segment (start 161.5 106) (end 159.58 106) (width 0.2) (layer "F.Cu") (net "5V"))
 (segment (start 158.25 85.33) (end 157.08 86.5) (width 0.2) (layer "F.Cu") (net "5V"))
 (segment (start 158.25 75.12) (end 158.25 85.33) (width 0.2) (layer "F.Cu") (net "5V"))
 (segment (start 159.58 106) (end 157.08 103.5) (width 0.2) (layer "F.Cu") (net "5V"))
 (segment (start 157.08 103.5) (end 157.08 86.5) (width 0.2) (layer "F.Cu") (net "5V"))
 (segment (start 142 60.5) (end 149 67.5) (width 0.2) (layer "F.Cu") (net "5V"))
 (via (at 149 67.5) (size 0.6) (drill 0.3) (layers "F.Cu" "B.Cu") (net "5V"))
 (segment (start 149 67.5) (end 156.62 75.12) (width 0.2) (layer "B.Cu") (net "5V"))
 (segment (start 156.62 75.12) (end 158.25 75.12) (width 0.2) (layer "B.Cu") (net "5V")))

